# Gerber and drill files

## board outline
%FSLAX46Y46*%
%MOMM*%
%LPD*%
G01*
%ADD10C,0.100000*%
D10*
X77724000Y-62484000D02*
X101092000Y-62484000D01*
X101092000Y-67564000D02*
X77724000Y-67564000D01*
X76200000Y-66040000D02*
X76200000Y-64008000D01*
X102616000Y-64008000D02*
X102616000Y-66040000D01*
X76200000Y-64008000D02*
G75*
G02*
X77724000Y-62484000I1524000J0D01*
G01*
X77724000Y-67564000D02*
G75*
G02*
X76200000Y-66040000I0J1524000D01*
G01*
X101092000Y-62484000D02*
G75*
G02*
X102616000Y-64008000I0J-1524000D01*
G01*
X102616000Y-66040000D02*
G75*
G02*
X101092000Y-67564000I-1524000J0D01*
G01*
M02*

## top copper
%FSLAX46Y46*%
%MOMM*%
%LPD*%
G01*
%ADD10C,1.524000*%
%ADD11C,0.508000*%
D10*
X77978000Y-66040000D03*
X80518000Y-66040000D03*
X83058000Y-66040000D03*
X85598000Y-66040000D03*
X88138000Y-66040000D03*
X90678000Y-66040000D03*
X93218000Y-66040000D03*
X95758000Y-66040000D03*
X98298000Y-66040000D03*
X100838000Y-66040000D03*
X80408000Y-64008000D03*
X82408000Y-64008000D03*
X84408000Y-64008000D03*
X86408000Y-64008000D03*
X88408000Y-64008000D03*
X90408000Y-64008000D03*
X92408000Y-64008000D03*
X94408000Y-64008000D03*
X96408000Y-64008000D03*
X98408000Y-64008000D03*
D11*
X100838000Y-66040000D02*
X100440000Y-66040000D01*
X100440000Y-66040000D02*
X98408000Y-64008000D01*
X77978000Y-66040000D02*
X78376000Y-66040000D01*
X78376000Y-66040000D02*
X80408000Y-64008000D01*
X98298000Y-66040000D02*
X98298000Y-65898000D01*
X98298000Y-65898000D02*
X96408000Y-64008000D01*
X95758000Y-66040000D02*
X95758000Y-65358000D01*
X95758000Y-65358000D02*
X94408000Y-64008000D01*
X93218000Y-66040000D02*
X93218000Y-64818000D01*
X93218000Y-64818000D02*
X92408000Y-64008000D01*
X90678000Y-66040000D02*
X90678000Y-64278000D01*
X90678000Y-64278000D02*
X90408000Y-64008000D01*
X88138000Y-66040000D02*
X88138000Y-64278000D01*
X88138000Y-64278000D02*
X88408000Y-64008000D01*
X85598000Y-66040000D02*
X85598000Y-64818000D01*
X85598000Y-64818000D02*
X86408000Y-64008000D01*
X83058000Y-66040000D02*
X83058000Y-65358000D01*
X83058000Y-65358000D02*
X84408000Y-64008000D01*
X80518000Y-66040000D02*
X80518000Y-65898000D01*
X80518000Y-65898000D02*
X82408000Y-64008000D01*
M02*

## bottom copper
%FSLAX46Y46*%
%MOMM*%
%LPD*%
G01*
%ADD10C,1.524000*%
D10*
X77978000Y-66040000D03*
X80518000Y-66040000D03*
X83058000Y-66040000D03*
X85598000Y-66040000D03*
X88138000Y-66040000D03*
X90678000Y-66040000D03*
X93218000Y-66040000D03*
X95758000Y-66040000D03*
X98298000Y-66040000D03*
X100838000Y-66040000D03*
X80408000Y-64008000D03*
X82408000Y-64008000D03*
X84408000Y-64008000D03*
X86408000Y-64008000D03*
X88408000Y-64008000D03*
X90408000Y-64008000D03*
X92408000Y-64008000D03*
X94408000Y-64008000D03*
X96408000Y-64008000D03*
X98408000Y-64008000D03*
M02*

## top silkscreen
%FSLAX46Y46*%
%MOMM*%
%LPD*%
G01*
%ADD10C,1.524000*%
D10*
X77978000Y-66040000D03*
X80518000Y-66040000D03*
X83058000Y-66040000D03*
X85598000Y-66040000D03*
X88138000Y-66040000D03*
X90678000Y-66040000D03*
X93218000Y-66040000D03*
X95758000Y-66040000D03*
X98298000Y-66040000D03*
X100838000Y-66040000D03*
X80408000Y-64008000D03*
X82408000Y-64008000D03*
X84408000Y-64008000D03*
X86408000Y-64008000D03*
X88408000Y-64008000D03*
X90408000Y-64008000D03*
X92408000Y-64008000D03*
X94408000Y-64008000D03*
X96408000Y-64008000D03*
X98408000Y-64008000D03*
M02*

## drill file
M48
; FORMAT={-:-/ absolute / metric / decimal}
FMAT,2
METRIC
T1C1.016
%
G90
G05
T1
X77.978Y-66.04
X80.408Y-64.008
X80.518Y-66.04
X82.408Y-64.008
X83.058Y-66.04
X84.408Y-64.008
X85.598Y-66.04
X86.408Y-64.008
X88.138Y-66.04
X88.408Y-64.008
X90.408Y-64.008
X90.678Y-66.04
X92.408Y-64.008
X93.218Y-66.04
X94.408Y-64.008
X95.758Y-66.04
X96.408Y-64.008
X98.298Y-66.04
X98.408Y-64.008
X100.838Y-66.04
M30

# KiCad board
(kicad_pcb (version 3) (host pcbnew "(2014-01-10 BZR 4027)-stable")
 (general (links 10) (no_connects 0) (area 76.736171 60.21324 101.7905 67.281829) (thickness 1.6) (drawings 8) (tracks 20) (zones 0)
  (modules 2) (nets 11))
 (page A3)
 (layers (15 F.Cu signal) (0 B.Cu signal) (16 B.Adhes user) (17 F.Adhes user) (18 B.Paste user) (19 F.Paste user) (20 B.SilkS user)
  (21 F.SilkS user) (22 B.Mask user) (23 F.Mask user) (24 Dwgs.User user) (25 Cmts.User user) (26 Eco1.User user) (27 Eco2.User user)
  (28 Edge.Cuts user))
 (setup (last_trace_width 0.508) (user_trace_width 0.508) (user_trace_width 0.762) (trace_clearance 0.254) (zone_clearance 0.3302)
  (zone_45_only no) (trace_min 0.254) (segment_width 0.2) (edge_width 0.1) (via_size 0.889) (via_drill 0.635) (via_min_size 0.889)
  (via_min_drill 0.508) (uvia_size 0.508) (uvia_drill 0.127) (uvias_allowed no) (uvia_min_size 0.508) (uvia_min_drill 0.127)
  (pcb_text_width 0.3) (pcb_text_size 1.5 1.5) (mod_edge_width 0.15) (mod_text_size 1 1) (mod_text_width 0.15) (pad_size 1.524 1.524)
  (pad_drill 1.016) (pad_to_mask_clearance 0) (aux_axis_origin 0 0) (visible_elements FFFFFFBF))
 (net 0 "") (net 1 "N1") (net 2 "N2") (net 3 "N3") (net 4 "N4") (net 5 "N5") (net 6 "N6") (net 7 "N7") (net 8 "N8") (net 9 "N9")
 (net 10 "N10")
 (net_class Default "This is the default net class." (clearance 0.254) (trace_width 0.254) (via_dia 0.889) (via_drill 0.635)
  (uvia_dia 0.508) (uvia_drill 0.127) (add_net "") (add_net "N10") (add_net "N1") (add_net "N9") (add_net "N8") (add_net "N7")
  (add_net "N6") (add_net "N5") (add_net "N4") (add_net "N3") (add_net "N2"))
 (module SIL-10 (layer F.Cu) (at 89.408 66.04)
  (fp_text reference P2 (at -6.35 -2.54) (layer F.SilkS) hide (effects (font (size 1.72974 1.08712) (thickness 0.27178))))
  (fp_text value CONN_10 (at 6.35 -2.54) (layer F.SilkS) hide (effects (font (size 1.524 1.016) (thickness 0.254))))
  (pad 1 thru_hole circle (at -11.43 0) (size 1.524 1.524) (drill 1.016) (layers *.Cu *.Mask F.SilkS) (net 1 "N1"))
  (pad 2 thru_hole circle (at -8.89 0) (size 1.524 1.524) (drill 1.016) (layers *.Cu *.Mask F.SilkS) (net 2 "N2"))
  (pad 3 thru_hole circle (at -6.35 0) (size 1.524 1.524) (drill 1.016) (layers *.Cu *.Mask F.SilkS) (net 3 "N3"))
  (pad 4 thru_hole circle (at -3.81 0) (size 1.524 1.524) (drill 1.016) (layers *.Cu *.Mask F.SilkS) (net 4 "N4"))
  (pad 5 thru_hole circle (at -1.27 0) (size 1.524 1.524) (drill 1.016) (layers *.Cu *.Mask F.SilkS) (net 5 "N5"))
  (pad 6 thru_hole circle (at 1.27 0) (size 1.524 1.524) (drill 1.016) (layers *.Cu *.Mask F.SilkS) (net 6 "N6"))
  (pad 7 thru_hole circle (at 3.81 0) (size 1.524 1.524) (drill 1.016) (layers *.Cu *.Mask F.SilkS) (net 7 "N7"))
  (pad 8 thru_hole circle (at 6.35 0) (size 1.524 1.524) (drill 1.016) (layers *.Cu *.Mask F.SilkS) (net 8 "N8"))
  (pad 9 thru_hole circle (at 8.89 0) (size 1.524 1.524) (drill 1.016) (layers *.Cu *.Mask F.SilkS) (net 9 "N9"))
  (pad 10 thru_hole circle (at 11.43 0) (size 1.524 1.524) (drill 1.016) (layers *.Cu *.Mask F.SilkS) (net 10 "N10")))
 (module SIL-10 (layer F.Cu) (at 89.408 64.008)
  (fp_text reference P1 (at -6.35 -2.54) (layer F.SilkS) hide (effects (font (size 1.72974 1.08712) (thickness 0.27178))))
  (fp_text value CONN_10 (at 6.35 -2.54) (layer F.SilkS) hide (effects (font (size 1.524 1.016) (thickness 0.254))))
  (pad 1 thru_hole circle (at -9 0) (size 1.524 1.524) (drill 1.016) (layers *.Cu *.Mask F.SilkS) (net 1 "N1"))
  (pad 2 thru_hole circle (at -7 0) (size 1.524 1.524) (drill 1.016) (layers *.Cu *.Mask F.SilkS) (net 2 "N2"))
  (pad 3 thru_hole circle (at -5 0) (size 1.524 1.524) (drill 1.016) (layers *.Cu *.Mask F.SilkS) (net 3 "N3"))
  (pad 4 thru_hole circle (at -3 0) (size 1.524 1.524) (drill 1.016) (layers *.Cu *.Mask F.SilkS) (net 4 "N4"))
  (pad 5 thru_hole circle (at -1 0) (size 1.524 1.524) (drill 1.016) (layers *.Cu *.Mask F.SilkS) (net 5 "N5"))
  (pad 6 thru_hole circle (at 1 0) (size 1.524 1.524) (drill 1.016) (layers *.Cu *.Mask F.SilkS) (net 6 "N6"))
  (pad 7 thru_hole circle (at 3 0) (size 1.524 1.524) (drill 1.016) (layers *.Cu *.Mask F.SilkS) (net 7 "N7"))
  (pad 8 thru_hole circle (at 5 0) (size 1.524 1.524) (drill 1.016) (layers *.Cu *.Mask F.SilkS) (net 8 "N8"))
  (pad 9 thru_hole circle (at 7 0) (size 1.524 1.524) (drill 1.016) (layers *.Cu *.Mask F.SilkS) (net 9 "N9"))
  (pad 10 thru_hole circle (at 9 0) (size 1.524 1.524) (drill 1.016) (layers *.Cu *.Mask F.SilkS) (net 10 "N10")))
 (gr_line (start 77.724 62.484) (end 101.092 62.484) (angle 90) (layer Edge.Cuts) (width 0.1))
 (gr_line (start 101.092 67.564) (end 77.724 67.564) (angle 90) (layer Edge.Cuts) (width 0.1))
 (gr_line (start 76.2 66.04) (end 76.2 64.008) (angle 90) (layer Edge.Cuts) (width 0.1))
 (gr_line (start 102.616 64.008) (end 102.616 66.04) (angle 90) (layer Edge.Cuts) (width 0.1))
 (gr_arc (start 77.724 64.008) (end 76.2 64.008) (angle 90) (layer Edge.Cuts) (width 0.1))
 (gr_arc (start 77.724 66.04) (end 77.724 67.564) (angle 90) (layer Edge.Cuts) (width 0.1))
 (gr_arc (start 101.092 64.008) (end 101.092 62.484) (angle 90) (layer Edge.Cuts) (width 0.1))
 (gr_arc (start 101.092 66.04) (end 102.616 66.04) (angle 90) (layer Edge.Cuts) (width 0.1))
 (segment (start 100.838 66.04) (end 100.44 66.04) (width 0.508) (layer F.Cu) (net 10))
 (segment (start 100.44 66.04) (end 98.408 64.008) (width 0.508) (layer F.Cu) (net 10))
 (segment (start 77.978 66.04) (end 78.376 66.04) (width 0.508) (layer F.Cu) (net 1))
 (segment (start 78.376 66.04) (end 80.408 64.008) (width 0.508) (layer F.Cu) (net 1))
 (segment (start 98.298 66.04) (end 98.298 65.898) (width 0.508) (layer F.Cu) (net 9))
 (segment (start 98.298 65.898) (end 96.408 64.008) (width 0.508) (layer F.Cu) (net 9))
 (segment (start 95.758 66.04) (end 95.758 65.358) (width 0.508) (layer F.Cu) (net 8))
 (segment (start 95.758 65.358) (end 94.408 64.008) (width 0.508) (layer F.Cu) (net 8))
 (segment (start 93.218 66.04) (end 93.218 64.818) (width 0.508) (layer F.Cu) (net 7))
 (segment (start 93.218 64.818) (end 92.408 64.008) (width 0.508) (layer F.Cu) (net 7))
 (segment (start 90.678 66.04) (end 90.678 64.278) (width 0.508) (layer F.Cu) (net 6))
 (segment (start 90.678 64.278) (end 90.408 64.008) (width 0.508) (layer F.Cu) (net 6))
 (segment (start 88.138 66.04) (end 88.138 64.278) (width 0.508) (layer F.Cu) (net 5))
 (segment (start 88.138 64.278) (end 88.408 64.008) (width 0.508) (layer F.Cu) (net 5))
 (segment (start 85.598 66.04) (end 85.598 64.818) (width 0.508) (layer F.Cu) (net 4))
 (segment (start 85.598 64.818) (end 86.408 64.008) (width 0.508) (layer F.Cu) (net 4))
 (segment (start 83.058 66.04) (end 83.058 65.358) (width 0.508) (layer F.Cu) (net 3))
 (segment (start 83.058 65.358) (end 84.408 64.008) (width 0.508) (layer F.Cu) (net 3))
 (segment (start 80.518 66.04) (end 80.518 65.898) (width 0.508) (layer F.Cu) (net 2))
 (segment (start 80.518 65.898) (end 82.408 64.008) (width 0.508) (layer F.Cu) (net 2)))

